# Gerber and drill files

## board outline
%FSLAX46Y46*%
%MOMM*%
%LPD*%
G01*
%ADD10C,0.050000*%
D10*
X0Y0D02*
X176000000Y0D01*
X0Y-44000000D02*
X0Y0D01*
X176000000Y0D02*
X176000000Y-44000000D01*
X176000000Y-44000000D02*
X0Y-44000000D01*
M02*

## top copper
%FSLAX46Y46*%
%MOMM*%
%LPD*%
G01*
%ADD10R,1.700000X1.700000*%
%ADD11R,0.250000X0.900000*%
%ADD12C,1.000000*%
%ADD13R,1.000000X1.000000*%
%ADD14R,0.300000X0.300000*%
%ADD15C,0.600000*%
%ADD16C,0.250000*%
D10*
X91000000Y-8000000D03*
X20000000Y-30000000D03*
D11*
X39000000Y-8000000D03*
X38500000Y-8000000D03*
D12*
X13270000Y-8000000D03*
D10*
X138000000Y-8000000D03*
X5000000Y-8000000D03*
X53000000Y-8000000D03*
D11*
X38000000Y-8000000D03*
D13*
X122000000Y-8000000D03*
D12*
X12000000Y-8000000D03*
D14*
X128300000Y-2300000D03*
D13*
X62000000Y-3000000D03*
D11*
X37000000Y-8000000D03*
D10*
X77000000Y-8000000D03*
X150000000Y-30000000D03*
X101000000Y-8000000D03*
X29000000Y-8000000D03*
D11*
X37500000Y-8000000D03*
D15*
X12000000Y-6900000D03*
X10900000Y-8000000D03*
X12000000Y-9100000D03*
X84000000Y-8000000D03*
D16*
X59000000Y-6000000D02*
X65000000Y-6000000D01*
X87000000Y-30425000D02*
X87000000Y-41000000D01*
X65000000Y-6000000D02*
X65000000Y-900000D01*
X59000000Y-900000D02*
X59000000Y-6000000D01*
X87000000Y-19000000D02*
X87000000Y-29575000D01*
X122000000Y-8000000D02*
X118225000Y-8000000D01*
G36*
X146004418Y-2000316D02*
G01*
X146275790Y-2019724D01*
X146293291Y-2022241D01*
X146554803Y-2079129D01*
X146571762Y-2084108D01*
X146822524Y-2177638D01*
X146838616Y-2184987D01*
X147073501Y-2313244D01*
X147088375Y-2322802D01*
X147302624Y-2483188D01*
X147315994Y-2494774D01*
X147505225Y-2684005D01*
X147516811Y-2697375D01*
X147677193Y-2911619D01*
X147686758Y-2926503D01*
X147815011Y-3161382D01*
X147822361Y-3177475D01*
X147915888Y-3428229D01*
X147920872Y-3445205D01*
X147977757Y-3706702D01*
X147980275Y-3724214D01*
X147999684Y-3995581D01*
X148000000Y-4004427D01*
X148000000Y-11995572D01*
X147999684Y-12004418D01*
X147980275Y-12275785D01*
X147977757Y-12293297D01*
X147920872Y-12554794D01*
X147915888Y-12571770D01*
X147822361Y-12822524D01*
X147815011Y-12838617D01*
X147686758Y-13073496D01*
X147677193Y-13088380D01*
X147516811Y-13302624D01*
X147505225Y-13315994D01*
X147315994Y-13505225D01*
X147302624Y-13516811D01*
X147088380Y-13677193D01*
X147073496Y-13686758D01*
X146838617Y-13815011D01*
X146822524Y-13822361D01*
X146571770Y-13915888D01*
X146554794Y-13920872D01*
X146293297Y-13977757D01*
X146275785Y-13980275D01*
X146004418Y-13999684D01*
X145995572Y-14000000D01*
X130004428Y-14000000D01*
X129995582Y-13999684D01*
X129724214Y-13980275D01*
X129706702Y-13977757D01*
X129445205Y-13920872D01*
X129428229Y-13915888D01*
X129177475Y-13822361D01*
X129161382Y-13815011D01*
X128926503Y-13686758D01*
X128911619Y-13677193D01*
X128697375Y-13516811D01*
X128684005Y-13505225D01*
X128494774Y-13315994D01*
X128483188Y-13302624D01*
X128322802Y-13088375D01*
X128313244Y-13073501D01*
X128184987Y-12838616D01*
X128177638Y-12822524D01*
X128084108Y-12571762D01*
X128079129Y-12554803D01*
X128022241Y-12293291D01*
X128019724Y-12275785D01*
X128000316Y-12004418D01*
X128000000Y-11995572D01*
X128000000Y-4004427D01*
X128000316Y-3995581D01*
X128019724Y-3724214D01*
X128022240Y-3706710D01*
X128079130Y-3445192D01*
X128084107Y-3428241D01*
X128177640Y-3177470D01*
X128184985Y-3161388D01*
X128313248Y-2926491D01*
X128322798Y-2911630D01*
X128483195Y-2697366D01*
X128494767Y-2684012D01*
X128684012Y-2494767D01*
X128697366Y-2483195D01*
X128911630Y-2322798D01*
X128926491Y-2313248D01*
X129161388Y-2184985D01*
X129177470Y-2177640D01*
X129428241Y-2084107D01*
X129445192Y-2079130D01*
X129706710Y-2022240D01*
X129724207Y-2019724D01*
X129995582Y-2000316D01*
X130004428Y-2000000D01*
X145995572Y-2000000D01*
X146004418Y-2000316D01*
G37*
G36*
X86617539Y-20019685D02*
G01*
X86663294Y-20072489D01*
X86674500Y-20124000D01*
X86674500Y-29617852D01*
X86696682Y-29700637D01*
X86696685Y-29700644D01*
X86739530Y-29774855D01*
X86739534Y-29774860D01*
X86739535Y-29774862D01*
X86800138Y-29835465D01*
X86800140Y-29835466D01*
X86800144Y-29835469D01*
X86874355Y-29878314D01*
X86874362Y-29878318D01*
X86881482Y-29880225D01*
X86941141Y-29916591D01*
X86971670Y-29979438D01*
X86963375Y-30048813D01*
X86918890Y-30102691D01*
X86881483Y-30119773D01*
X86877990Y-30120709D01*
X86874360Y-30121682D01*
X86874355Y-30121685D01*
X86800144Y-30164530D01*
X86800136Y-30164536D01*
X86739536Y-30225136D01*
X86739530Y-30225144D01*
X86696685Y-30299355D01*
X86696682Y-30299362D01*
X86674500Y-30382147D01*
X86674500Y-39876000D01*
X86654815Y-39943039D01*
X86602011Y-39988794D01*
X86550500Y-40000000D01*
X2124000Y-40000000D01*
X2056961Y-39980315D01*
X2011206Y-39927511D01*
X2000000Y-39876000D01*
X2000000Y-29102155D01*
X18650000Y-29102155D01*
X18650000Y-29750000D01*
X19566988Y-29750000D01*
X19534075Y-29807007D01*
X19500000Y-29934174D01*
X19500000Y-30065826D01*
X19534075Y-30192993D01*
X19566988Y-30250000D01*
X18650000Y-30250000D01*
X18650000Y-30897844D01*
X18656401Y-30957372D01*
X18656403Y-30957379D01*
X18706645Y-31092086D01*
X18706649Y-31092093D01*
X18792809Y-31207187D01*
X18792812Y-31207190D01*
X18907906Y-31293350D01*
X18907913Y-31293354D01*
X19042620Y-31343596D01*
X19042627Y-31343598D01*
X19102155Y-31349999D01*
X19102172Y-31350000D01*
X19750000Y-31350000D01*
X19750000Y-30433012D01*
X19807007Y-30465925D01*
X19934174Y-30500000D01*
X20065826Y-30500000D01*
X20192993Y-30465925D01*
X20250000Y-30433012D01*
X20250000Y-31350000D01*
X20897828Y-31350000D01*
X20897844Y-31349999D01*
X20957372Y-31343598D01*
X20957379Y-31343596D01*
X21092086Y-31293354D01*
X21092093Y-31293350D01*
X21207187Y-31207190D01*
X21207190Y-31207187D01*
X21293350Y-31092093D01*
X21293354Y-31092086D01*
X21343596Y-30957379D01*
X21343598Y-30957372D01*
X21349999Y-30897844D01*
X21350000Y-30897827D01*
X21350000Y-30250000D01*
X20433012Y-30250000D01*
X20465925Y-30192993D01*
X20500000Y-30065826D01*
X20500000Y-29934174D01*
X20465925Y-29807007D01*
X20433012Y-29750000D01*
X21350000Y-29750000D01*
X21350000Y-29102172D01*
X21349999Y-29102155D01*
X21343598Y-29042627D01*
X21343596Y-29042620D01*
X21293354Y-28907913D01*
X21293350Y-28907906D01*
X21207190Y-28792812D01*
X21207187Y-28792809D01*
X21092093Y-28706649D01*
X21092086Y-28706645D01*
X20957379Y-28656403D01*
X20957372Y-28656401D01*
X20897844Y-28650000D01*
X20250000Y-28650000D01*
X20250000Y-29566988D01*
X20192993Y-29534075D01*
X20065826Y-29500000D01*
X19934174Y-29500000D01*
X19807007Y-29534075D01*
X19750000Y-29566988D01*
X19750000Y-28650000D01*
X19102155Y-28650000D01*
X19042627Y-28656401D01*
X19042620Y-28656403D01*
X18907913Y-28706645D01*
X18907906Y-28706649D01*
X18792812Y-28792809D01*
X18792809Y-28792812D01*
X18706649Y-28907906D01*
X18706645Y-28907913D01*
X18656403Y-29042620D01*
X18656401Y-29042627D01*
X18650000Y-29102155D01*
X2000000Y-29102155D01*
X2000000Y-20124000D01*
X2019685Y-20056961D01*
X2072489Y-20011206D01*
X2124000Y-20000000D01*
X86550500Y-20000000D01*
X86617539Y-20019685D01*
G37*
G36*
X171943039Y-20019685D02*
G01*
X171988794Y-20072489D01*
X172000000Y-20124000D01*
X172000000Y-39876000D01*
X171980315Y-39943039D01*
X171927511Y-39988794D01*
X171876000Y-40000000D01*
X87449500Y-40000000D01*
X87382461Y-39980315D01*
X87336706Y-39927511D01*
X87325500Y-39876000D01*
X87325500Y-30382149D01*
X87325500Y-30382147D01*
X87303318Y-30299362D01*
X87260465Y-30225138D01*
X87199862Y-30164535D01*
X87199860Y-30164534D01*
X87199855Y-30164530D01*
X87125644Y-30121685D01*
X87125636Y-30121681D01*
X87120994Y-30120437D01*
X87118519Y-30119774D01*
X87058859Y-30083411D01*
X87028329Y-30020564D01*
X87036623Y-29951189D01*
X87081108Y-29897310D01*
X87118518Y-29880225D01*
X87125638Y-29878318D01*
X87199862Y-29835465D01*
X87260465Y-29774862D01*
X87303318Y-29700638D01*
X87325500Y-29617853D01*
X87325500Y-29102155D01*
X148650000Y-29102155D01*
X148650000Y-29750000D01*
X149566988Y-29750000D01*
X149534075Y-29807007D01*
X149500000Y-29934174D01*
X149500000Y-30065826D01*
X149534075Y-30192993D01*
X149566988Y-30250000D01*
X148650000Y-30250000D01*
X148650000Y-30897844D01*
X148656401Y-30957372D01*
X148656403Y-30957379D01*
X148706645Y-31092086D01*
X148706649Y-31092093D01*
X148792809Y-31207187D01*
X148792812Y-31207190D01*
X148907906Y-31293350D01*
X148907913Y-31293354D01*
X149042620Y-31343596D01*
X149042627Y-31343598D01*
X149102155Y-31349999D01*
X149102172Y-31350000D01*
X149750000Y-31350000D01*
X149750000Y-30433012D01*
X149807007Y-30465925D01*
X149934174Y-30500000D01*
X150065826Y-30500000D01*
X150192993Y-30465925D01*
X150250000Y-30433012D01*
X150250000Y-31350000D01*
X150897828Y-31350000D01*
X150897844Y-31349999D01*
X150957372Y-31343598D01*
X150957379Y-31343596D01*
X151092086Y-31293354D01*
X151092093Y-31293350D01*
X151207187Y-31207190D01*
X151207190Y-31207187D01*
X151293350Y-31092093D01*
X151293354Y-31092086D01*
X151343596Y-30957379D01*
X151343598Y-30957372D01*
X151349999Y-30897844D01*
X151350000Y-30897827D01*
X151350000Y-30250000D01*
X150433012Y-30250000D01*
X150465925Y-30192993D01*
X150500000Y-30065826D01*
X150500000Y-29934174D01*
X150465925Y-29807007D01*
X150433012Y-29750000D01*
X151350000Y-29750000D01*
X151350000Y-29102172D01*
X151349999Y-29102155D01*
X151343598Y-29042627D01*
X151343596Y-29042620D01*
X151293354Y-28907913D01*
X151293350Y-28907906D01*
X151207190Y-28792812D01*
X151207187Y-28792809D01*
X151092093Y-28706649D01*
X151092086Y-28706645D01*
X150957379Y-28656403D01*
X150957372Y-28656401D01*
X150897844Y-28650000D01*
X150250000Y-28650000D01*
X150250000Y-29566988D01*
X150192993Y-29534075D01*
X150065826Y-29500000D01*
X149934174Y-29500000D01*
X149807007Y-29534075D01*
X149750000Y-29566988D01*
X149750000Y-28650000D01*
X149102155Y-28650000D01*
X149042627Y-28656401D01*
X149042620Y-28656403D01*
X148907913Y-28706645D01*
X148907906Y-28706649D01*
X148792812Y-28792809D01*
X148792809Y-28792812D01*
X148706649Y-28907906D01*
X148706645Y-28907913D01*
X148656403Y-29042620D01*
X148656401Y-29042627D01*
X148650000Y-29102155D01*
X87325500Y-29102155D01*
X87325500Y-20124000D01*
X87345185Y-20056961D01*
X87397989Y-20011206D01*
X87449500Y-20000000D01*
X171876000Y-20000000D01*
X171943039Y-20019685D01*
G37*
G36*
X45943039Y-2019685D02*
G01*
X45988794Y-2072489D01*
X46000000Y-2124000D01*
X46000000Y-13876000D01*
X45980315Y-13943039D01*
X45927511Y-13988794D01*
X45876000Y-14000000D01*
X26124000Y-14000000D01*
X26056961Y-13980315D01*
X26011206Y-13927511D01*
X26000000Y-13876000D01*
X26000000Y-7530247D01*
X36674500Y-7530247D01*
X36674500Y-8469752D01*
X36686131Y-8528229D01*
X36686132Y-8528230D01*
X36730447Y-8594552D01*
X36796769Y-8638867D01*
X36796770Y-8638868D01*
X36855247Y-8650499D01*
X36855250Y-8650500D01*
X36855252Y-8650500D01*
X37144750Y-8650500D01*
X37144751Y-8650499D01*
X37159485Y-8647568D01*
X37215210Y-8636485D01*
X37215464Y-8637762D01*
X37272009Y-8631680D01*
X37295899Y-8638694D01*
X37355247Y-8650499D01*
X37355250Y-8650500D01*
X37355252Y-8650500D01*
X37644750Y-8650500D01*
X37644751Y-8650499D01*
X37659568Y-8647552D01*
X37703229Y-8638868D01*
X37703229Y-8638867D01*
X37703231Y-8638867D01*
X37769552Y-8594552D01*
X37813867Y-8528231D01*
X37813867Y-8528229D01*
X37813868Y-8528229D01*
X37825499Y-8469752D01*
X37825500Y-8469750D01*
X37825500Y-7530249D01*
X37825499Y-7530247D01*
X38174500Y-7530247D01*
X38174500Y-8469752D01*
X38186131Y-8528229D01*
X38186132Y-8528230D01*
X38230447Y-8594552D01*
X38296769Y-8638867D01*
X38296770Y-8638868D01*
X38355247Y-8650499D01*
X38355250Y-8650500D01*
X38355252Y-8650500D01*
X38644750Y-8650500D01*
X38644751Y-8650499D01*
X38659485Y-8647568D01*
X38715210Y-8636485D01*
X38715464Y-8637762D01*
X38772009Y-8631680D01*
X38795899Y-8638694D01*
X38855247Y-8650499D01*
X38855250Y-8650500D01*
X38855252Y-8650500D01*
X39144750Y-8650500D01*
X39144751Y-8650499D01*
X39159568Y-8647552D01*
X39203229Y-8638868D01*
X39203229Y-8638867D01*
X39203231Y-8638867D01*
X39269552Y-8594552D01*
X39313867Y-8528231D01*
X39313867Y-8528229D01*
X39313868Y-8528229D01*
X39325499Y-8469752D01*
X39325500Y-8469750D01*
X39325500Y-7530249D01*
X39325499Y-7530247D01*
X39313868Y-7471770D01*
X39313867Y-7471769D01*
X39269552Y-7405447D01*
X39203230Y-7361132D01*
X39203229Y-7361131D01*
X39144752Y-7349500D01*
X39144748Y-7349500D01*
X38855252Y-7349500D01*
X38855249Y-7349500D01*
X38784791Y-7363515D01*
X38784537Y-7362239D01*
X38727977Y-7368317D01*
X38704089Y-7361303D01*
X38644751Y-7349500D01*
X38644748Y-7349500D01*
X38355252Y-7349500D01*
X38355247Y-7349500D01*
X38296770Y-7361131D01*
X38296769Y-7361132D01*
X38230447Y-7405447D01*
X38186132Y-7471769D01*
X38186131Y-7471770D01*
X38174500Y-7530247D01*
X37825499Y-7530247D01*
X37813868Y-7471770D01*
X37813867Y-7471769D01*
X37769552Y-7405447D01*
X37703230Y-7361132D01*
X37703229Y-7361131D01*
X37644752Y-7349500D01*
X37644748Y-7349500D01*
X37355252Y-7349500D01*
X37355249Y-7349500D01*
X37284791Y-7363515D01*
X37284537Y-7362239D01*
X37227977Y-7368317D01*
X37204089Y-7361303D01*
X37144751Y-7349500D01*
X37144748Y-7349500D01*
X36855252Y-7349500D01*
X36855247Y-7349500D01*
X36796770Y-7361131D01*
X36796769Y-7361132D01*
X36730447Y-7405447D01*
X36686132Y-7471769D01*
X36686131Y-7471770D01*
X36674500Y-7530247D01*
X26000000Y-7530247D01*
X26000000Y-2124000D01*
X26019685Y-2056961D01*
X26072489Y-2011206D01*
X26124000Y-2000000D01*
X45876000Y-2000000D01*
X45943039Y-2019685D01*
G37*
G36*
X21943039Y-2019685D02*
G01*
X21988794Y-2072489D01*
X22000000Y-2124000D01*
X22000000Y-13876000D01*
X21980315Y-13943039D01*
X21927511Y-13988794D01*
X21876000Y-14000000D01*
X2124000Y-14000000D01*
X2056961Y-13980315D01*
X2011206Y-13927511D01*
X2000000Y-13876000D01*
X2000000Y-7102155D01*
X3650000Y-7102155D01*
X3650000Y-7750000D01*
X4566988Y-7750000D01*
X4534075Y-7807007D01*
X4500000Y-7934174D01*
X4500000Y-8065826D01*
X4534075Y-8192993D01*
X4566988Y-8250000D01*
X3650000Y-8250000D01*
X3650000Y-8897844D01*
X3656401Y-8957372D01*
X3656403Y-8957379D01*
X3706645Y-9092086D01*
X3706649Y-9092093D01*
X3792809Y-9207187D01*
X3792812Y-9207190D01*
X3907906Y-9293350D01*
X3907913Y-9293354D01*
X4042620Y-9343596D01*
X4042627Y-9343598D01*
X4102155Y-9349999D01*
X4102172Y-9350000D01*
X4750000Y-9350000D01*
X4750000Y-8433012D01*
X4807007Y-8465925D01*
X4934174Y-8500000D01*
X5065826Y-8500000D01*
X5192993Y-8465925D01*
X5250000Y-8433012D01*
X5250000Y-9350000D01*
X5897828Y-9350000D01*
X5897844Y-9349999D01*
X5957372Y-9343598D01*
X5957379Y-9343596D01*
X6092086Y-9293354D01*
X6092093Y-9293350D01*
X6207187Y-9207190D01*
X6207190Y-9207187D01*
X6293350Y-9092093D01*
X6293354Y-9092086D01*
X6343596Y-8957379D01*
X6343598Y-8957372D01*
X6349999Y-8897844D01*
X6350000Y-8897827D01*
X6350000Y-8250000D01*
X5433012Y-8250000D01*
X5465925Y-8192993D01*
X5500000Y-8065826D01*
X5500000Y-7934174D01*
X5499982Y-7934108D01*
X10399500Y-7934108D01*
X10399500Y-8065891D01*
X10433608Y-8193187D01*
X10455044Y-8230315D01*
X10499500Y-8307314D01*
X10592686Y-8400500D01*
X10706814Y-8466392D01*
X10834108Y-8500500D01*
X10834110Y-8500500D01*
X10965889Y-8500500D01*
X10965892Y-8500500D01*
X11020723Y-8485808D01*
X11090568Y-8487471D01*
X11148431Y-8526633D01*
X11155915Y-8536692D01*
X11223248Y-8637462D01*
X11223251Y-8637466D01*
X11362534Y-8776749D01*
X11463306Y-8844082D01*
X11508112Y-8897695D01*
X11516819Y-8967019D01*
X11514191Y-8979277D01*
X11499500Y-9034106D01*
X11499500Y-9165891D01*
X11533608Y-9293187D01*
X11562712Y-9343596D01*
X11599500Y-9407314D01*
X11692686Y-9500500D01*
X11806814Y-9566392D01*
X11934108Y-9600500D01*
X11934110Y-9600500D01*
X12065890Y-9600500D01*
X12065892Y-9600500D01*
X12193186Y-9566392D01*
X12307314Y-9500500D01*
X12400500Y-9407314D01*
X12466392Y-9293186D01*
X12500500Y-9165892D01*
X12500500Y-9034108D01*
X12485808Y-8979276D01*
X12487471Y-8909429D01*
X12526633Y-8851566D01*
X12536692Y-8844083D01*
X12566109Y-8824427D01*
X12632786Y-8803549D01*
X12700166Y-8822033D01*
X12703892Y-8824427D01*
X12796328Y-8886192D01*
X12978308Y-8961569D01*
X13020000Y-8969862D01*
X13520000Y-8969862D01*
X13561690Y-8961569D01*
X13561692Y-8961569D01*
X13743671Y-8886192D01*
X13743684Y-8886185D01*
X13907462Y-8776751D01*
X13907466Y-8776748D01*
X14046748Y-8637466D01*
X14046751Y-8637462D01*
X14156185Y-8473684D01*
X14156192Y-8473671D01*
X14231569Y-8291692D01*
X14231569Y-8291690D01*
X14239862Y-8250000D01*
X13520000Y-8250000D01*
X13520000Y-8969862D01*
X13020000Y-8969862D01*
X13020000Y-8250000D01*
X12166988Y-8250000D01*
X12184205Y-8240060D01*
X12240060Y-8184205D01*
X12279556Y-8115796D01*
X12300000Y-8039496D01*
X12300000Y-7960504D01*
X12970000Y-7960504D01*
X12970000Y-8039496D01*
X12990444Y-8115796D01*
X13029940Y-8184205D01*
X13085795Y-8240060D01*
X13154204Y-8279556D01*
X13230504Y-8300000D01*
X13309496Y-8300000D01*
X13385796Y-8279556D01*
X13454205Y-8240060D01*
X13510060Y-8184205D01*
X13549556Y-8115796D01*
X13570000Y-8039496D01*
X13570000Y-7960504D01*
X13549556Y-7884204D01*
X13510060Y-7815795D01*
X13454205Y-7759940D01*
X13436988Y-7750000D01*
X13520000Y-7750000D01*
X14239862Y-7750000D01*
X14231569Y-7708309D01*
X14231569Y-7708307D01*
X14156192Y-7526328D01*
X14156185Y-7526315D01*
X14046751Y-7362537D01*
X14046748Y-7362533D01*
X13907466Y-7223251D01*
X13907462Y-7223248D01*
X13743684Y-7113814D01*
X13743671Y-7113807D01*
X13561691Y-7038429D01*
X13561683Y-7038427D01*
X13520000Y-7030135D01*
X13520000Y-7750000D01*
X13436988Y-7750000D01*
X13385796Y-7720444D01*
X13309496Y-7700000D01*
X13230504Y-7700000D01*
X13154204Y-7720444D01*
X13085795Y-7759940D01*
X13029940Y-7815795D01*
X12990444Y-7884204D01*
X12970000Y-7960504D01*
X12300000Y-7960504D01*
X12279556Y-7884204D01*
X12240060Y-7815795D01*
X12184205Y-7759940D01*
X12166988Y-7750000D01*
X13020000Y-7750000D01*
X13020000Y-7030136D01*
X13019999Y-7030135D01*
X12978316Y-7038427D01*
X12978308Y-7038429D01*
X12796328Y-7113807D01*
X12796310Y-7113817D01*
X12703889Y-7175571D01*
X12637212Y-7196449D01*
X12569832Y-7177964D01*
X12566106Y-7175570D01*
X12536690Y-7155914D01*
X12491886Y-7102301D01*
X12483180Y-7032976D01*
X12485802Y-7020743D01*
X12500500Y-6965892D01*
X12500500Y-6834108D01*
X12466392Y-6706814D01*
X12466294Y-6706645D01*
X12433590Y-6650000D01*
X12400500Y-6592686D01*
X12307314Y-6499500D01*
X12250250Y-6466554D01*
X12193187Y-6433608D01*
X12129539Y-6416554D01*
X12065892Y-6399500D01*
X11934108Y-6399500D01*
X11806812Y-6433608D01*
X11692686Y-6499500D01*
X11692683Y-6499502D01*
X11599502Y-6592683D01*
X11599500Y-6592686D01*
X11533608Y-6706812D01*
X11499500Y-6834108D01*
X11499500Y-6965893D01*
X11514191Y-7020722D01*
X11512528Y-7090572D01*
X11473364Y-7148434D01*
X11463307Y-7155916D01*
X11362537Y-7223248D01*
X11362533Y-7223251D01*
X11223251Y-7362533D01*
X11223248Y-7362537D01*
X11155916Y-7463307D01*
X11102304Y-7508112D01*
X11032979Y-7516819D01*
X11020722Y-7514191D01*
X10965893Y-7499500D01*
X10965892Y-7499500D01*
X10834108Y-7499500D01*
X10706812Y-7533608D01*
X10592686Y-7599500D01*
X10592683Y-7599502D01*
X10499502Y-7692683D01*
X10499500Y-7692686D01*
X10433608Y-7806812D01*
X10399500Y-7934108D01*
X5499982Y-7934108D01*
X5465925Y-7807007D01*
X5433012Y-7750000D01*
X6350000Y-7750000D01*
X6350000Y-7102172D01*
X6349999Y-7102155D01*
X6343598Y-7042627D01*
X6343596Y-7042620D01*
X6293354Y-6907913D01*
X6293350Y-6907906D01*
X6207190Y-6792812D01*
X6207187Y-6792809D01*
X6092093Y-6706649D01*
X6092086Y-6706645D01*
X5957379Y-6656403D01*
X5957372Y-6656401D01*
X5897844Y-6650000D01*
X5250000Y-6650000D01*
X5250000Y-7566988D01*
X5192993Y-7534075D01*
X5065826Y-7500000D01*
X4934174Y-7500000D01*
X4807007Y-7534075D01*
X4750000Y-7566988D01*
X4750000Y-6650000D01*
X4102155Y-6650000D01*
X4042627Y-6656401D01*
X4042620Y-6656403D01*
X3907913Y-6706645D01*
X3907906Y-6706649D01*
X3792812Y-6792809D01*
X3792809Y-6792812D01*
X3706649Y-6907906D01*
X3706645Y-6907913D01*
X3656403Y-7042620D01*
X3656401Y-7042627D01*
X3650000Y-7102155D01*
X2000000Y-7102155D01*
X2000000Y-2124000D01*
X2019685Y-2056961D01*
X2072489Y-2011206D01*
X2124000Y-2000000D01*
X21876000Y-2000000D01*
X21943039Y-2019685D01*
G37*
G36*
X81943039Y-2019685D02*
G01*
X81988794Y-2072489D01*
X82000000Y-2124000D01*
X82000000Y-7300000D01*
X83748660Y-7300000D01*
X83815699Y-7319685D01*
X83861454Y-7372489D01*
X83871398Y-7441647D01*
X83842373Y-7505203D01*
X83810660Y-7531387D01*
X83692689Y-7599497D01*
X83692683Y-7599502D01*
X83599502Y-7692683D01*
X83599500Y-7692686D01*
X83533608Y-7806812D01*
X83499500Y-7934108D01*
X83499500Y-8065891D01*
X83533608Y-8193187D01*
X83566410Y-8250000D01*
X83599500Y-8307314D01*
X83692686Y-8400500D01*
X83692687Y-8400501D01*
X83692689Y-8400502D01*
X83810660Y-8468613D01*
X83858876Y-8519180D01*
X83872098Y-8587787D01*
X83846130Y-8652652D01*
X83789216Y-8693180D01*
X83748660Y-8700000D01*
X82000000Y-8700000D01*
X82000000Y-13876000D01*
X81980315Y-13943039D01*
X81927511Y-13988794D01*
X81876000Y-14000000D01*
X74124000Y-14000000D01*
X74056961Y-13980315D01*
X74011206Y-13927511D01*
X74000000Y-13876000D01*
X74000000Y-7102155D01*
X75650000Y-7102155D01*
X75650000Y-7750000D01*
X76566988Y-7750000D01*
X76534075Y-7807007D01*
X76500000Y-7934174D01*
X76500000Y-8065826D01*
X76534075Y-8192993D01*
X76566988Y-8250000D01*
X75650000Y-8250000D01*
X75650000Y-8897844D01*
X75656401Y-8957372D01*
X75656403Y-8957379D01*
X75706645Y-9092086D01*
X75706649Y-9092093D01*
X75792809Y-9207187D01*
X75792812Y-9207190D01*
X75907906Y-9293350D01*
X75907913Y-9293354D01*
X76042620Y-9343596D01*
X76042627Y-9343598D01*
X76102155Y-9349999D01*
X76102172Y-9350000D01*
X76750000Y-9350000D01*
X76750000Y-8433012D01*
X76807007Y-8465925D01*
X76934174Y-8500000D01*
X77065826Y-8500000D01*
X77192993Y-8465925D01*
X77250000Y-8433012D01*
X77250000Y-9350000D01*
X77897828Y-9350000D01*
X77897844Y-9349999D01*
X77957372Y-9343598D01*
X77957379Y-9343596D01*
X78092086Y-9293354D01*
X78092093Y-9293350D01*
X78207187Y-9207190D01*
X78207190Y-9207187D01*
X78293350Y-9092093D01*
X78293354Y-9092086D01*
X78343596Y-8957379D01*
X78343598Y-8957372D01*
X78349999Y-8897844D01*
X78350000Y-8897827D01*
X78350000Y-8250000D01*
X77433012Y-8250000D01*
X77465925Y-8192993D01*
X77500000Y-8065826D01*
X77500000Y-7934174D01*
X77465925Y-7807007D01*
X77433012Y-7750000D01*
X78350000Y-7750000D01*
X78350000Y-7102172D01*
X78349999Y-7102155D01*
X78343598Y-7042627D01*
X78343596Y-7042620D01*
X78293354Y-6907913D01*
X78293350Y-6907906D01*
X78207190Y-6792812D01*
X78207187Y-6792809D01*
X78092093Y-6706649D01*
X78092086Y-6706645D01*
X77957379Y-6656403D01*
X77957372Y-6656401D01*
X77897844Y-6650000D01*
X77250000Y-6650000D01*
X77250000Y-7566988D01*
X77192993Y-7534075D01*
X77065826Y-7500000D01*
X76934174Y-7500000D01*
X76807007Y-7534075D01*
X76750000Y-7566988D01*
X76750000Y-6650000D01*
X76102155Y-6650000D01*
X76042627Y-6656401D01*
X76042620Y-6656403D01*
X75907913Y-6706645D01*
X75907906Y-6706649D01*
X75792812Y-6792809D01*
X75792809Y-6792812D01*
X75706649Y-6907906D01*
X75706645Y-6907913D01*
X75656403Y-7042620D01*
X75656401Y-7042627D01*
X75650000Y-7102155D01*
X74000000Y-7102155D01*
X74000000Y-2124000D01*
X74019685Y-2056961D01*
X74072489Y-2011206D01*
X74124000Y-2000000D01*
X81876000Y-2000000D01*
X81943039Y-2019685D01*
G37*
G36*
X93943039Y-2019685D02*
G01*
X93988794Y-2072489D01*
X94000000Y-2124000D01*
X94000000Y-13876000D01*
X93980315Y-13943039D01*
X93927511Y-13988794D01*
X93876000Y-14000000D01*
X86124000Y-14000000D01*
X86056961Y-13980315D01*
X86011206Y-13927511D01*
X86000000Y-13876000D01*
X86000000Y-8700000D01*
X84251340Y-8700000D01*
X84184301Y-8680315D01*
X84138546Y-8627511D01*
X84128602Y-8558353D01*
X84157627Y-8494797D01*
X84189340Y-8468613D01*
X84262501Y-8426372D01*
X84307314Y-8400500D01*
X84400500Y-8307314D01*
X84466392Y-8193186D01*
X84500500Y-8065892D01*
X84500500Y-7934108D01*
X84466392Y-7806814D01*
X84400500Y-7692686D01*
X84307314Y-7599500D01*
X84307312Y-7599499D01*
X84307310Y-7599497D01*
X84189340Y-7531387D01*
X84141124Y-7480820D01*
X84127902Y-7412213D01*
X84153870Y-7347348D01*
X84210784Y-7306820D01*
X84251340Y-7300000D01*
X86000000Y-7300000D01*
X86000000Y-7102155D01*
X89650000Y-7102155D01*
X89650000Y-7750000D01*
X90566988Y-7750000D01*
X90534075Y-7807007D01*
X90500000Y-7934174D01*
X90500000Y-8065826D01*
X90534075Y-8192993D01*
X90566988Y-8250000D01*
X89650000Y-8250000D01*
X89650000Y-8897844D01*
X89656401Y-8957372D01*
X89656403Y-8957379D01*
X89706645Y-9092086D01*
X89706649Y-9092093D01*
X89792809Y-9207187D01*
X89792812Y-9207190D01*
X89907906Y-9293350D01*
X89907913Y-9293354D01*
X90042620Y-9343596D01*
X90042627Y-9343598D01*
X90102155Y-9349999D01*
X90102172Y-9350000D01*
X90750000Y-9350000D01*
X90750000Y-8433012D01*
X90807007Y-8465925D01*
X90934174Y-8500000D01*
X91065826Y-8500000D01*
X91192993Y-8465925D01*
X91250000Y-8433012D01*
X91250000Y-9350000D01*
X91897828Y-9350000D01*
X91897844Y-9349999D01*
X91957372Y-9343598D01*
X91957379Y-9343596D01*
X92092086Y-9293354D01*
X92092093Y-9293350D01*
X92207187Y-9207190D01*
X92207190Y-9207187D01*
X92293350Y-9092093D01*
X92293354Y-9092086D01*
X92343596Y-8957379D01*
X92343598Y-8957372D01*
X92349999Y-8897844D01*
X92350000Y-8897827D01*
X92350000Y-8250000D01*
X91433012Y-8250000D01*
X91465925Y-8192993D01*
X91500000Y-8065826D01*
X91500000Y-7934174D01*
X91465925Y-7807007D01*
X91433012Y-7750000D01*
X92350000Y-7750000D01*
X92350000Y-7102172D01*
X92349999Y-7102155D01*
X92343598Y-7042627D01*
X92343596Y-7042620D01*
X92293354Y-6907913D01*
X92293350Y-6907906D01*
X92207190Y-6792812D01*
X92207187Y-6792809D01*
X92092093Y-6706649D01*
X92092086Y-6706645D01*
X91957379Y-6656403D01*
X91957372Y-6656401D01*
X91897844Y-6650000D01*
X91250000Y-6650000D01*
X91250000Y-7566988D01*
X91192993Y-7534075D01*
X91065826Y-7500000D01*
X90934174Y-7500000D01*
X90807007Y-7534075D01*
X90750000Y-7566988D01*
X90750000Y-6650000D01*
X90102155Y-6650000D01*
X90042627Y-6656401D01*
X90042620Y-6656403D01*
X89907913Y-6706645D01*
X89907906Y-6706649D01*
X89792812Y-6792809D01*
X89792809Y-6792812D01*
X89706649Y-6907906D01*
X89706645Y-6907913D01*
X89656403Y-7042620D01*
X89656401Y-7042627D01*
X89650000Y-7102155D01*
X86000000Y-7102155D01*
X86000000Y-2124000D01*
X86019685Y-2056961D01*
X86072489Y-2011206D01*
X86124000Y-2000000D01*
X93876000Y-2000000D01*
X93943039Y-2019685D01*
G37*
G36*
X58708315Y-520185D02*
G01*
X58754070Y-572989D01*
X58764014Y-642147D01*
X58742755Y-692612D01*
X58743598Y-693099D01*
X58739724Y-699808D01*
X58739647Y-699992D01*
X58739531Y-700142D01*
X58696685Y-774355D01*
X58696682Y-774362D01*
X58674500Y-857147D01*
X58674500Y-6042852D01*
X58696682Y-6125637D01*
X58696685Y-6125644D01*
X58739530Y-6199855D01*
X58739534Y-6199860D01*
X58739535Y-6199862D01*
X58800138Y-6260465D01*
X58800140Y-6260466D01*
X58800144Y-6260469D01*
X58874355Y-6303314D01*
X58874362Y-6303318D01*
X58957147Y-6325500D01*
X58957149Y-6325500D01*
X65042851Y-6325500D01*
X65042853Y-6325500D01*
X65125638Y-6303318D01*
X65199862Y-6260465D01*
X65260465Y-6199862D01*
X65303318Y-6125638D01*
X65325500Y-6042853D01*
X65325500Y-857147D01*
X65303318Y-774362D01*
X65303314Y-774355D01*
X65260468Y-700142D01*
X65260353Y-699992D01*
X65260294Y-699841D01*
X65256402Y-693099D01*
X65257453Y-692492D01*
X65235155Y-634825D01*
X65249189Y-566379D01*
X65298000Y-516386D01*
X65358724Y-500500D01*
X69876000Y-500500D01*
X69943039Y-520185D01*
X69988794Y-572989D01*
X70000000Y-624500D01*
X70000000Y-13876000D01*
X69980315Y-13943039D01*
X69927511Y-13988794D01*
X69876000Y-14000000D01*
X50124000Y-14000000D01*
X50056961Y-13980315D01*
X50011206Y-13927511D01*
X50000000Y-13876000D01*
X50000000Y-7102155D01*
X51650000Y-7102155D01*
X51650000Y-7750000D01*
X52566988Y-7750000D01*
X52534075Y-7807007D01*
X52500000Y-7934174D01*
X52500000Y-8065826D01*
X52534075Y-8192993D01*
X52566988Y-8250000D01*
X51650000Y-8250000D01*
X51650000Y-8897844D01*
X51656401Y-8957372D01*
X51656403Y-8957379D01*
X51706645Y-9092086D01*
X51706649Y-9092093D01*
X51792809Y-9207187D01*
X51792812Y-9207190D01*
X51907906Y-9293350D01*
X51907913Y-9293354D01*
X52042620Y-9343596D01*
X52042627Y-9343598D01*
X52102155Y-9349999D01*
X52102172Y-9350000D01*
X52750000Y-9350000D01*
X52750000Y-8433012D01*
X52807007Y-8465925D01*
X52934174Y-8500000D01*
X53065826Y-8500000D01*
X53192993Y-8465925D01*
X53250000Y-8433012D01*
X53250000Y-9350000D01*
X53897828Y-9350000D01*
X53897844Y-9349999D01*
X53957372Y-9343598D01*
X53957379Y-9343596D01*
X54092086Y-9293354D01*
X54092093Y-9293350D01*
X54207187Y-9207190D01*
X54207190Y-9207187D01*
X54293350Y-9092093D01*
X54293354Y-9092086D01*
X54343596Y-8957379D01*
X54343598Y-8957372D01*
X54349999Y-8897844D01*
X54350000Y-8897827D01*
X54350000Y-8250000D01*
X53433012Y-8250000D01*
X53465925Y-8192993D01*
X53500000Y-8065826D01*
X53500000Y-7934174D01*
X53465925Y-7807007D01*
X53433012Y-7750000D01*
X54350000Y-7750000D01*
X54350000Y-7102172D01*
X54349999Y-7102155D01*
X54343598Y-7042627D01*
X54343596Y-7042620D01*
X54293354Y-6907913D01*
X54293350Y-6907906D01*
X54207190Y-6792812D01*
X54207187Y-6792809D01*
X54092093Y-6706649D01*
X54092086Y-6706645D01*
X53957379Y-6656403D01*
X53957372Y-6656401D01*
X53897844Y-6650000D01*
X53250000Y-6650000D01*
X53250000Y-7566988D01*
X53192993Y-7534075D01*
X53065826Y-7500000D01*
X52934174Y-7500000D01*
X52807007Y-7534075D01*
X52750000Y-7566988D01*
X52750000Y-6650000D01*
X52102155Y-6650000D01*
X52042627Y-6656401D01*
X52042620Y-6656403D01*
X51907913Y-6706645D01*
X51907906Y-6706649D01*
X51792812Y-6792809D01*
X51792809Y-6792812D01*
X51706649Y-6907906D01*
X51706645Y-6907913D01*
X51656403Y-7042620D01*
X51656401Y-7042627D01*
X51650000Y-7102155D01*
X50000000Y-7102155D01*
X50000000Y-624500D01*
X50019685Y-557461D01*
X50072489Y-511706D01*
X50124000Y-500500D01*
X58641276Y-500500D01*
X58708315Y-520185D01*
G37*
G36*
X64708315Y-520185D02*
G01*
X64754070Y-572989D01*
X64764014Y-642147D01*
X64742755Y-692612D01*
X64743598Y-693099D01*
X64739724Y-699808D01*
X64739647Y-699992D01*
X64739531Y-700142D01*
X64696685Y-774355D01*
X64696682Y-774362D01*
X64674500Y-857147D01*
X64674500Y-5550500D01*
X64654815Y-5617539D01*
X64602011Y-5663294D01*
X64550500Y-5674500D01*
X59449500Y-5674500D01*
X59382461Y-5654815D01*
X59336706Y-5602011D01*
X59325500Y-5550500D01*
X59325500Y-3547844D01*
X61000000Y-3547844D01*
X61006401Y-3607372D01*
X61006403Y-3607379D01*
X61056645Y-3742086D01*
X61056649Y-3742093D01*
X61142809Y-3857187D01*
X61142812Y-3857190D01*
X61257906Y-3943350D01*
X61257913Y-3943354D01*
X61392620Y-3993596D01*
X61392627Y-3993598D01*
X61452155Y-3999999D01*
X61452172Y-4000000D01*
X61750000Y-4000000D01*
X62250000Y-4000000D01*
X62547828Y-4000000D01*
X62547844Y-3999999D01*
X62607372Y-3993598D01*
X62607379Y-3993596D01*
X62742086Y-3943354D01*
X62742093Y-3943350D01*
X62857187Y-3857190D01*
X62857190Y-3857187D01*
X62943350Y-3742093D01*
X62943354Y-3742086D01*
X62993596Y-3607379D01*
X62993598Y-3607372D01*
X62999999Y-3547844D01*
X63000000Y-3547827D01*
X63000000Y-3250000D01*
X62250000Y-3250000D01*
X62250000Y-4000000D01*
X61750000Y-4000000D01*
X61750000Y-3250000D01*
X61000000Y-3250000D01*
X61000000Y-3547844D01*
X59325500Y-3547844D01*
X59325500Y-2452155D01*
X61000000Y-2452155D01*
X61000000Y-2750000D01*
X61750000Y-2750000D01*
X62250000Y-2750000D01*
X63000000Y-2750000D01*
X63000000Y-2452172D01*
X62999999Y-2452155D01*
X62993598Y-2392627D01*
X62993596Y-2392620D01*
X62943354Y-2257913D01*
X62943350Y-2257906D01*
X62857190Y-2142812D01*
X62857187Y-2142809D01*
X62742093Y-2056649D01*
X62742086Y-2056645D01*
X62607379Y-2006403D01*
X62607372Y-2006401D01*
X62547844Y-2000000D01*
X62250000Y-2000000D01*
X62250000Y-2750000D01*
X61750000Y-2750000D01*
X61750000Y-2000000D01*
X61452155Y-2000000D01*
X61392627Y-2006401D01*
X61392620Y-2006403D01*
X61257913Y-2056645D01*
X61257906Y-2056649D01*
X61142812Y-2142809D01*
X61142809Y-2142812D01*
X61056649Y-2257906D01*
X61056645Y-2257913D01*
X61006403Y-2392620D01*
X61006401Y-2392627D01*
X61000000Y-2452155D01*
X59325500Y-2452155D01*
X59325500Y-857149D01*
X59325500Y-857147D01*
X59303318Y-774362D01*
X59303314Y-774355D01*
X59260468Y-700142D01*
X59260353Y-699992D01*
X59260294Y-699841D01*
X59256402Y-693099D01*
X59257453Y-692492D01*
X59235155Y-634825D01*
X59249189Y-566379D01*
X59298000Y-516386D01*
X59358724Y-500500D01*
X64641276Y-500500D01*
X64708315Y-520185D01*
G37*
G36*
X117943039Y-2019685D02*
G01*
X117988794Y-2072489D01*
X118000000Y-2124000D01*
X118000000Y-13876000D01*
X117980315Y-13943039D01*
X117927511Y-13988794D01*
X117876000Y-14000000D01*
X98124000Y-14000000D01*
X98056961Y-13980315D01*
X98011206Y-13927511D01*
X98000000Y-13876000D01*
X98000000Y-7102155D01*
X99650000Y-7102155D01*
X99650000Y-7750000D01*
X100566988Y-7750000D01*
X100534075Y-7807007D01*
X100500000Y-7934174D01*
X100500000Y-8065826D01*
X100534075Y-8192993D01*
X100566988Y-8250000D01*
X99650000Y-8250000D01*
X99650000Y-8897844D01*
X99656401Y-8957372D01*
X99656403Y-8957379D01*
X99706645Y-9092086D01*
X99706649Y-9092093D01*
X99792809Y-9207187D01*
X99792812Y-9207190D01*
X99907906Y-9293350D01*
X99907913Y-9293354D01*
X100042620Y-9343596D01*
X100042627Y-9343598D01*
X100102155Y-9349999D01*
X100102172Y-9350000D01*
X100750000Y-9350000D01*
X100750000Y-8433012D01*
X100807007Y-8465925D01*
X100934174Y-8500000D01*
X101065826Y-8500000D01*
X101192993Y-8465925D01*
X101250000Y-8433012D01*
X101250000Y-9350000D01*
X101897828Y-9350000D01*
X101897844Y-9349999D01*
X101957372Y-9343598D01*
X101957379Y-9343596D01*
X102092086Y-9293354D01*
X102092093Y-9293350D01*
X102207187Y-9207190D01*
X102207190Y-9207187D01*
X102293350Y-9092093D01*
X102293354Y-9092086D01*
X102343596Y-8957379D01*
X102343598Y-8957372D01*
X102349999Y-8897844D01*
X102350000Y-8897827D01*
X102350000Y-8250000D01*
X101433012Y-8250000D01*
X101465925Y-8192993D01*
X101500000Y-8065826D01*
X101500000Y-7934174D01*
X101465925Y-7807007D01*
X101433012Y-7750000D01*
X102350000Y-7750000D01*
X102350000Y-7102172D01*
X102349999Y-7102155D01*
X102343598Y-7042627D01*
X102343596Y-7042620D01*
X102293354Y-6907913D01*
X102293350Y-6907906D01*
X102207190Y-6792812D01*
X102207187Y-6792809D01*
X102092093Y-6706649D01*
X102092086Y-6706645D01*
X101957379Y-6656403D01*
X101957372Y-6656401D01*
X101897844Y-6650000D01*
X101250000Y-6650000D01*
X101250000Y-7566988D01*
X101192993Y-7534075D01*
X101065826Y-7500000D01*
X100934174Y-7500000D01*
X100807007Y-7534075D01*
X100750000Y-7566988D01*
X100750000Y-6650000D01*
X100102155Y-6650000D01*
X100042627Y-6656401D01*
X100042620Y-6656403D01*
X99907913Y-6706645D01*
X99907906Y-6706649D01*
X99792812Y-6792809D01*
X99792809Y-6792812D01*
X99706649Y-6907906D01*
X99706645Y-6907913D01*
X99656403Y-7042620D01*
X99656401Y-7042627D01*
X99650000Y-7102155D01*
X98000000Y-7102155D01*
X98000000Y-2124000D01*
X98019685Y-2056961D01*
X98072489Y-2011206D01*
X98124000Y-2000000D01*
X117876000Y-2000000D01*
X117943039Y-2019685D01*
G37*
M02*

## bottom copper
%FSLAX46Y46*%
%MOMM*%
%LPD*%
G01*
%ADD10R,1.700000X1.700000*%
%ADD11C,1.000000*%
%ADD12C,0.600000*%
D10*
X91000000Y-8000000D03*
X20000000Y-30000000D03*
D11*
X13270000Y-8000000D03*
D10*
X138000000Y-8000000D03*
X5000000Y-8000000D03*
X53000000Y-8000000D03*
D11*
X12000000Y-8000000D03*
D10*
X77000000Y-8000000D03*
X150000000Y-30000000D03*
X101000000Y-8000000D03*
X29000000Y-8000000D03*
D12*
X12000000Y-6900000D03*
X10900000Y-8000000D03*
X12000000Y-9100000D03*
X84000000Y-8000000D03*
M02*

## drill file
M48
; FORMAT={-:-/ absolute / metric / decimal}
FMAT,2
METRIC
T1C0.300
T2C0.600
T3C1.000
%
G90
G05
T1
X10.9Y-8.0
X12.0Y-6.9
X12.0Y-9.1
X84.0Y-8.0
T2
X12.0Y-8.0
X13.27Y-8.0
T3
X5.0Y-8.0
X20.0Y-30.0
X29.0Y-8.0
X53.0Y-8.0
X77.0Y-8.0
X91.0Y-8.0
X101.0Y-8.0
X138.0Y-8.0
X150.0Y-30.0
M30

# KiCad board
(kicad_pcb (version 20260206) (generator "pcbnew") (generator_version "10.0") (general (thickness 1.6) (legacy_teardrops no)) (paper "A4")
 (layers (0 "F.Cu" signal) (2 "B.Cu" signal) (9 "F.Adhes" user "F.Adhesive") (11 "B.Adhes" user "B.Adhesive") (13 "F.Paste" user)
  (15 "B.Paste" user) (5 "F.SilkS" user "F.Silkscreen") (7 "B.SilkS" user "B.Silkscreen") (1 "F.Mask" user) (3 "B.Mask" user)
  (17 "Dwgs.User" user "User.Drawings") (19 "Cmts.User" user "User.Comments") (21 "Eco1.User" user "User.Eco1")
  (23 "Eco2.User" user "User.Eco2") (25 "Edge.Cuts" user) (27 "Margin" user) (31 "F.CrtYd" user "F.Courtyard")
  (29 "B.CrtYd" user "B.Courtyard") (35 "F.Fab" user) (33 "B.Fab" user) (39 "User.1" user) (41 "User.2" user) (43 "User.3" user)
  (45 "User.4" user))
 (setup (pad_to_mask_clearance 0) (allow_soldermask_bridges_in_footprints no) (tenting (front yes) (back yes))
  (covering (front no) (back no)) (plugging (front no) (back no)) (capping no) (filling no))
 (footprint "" (layer "F.Cu") (at 91 8)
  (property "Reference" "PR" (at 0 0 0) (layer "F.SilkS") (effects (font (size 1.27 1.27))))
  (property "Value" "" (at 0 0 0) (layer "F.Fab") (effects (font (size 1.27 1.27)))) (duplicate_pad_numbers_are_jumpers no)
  (pad "1" thru_hole rect (at 0 0) (size 1.7 1.7) (drill 1) (layers "*.Cu" "*.Mask") (remove_unused_layers no) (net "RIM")))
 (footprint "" (layer "F.Cu") (at 20 30)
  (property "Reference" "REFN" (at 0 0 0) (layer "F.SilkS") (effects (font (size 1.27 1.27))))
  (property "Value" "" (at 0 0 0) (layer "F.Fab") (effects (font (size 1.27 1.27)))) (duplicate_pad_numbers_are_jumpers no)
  (pad "1" thru_hole rect (at 0 0) (size 1.7 1.7) (drill 1) (layers "*.Cu" "*.Mask") (remove_unused_layers no) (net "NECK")))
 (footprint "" (layer "F.Cu") (at 39 8)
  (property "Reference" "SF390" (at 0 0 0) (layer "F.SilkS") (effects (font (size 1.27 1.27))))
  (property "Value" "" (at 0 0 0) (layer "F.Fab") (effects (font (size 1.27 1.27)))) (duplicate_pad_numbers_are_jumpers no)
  (pad "1" smd rect (at 0 0) (size 0.25 0.9) (layers "F.Cu" "F.Mask" "F.Paste") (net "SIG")))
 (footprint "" (layer "F.Cu") (at 38.5 8)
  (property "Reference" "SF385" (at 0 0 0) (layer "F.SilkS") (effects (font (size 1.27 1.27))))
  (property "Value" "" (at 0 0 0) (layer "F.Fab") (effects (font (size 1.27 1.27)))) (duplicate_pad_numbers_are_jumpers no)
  (pad "1" smd rect (at 0 0) (size 0.25 0.9) (layers "F.Cu" "F.Mask" "F.Paste") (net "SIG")))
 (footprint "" (layer "F.Cu") (at 13.27 8)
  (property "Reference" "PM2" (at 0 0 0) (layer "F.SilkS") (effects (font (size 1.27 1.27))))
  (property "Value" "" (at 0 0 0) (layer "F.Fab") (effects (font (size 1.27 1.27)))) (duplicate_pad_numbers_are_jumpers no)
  (pad "1" thru_hole circle (at 0 0) (size 1 1) (drill 0.6) (layers "*.Cu" "*.Mask") (remove_unused_layers no) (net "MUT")
   (thermal_bridge_angle 90)))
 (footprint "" (layer "F.Cu") (at 138 8)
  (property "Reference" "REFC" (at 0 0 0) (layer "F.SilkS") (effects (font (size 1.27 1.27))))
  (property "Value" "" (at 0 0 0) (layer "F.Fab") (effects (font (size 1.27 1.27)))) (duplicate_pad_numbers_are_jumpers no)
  (pad "1" thru_hole rect (at 0 0) (size 1.7 1.7) (drill 1) (layers "*.Cu" "*.Mask") (remove_unused_layers no) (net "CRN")))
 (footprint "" (layer "F.Cu") (at 5 8)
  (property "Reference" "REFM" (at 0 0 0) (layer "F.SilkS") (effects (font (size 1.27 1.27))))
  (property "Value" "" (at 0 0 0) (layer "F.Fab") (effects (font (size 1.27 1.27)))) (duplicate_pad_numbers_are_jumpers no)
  (pad "1" thru_hole rect (at 0 0) (size 1.7 1.7) (drill 1) (layers "*.Cu" "*.Mask") (remove_unused_layers no) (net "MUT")))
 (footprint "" (layer "F.Cu") (at 53 8)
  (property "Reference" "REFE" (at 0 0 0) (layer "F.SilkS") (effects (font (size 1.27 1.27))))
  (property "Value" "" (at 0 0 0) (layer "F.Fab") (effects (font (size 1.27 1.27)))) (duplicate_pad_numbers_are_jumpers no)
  (pad "1" thru_hole rect (at 0 0) (size 1.7 1.7) (drill 1) (layers "*.Cu" "*.Mask") (remove_unused_layers no) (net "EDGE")))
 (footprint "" (layer "F.Cu") (at 38 8)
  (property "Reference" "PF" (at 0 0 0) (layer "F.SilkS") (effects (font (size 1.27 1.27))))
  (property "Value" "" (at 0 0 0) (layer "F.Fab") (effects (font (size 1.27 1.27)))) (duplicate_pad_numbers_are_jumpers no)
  (pad "1" smd rect (at 0 0) (size 0.25 0.9) (layers "F.Cu" "F.Mask" "F.Paste") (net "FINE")))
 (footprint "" (layer "F.Cu") (at 122 8)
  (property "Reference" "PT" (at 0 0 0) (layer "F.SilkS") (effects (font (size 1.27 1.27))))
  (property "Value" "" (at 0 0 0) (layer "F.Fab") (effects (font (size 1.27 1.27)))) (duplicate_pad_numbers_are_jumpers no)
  (pad "1" smd rect (at 0 0) (size 1 1) (layers "F.Cu" "F.Mask" "F.Paste") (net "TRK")))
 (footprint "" (layer "F.Cu") (at 12 8)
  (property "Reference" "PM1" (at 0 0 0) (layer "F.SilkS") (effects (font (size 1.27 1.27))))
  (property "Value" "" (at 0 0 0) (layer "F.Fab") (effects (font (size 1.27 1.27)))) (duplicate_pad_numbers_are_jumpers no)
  (pad "1" thru_hole circle (at 0 0) (size 1 1) (drill 0.6) (layers "*.Cu" "*.Mask") (remove_unused_layers no) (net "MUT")
   (thermal_bridge_angle 90)))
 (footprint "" (layer "F.Cu") (at 128.3 2.3)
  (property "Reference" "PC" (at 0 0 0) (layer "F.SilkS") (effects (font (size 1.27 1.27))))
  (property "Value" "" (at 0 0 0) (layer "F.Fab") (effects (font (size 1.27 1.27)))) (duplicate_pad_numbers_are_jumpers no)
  (pad "1" smd rect (at 0 0) (size 0.3 0.3) (layers "F.Cu" "F.Mask" "F.Paste") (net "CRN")))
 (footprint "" (layer "F.Cu") (at 62 3)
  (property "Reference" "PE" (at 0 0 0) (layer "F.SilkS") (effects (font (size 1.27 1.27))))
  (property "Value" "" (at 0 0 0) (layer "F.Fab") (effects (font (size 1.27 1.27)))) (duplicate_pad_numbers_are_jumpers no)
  (pad "1" smd rect (at 0 0) (size 1 1) (layers "F.Cu" "F.Mask" "F.Paste") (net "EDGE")))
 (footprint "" (layer "F.Cu") (at 37 8)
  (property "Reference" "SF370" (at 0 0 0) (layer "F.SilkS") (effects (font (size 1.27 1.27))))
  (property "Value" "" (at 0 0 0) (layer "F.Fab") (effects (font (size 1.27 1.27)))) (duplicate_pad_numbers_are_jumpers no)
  (pad "1" smd rect (at 0 0) (size 0.25 0.9) (layers "F.Cu" "F.Mask" "F.Paste") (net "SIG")))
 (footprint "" (layer "F.Cu") (at 77 8)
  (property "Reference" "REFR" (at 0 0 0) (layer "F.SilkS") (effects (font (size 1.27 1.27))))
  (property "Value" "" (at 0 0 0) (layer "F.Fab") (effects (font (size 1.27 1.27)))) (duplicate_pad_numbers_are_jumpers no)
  (pad "1" thru_hole rect (at 0 0) (size 1.7 1.7) (drill 1) (layers "*.Cu" "*.Mask") (remove_unused_layers no) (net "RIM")))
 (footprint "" (layer "F.Cu") (at 150 30)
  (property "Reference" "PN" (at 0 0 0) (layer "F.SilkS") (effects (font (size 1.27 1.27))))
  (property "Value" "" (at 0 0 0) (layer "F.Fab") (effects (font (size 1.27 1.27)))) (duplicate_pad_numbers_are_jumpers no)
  (pad "1" thru_hole rect (at 0 0) (size 1.7 1.7) (drill 1) (layers "*.Cu" "*.Mask") (remove_unused_layers no) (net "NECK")))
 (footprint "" (layer "F.Cu") (at 101 8)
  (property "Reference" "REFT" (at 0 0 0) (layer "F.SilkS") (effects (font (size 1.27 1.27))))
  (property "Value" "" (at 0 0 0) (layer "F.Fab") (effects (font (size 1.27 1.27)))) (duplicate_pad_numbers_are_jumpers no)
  (pad "1" thru_hole rect (at 0 0) (size 1.7 1.7) (drill 1) (layers "*.Cu" "*.Mask") (remove_unused_layers no) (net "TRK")))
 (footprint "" (layer "F.Cu") (at 29 8)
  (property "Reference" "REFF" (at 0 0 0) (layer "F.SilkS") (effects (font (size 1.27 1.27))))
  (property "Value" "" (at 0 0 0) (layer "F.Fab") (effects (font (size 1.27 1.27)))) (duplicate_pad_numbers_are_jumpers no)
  (pad "1" thru_hole rect (at 0 0) (size 1.7 1.7) (drill 1) (layers "*.Cu" "*.Mask") (remove_unused_layers no) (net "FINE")))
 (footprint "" (layer "F.Cu") (at 37.5 8)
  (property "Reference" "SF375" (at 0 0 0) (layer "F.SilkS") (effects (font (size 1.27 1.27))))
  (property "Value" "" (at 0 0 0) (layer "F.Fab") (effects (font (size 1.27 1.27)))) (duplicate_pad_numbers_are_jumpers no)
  (pad "1" smd rect (at 0 0) (size 0.25 0.9) (layers "F.Cu" "F.Mask" "F.Paste") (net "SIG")))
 (gr_line (start 0 0) (end 176 0) (stroke (width 0.05) (type default)) (layer "Edge.Cuts"))
 (gr_line (start 0 44) (end 0 0) (stroke (width 0.05) (type default)) (layer "Edge.Cuts"))
 (gr_line (start 176 0) (end 176 44) (stroke (width 0.05) (type default)) (layer "Edge.Cuts"))
 (gr_line (start 176 44) (end 0 44) (stroke (width 0.05) (type default)) (layer "Edge.Cuts"))
 (segment (start 59 6) (end 65 6) (width 0.25) (layer "F.Cu") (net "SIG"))
 (segment (start 87 30.425) (end 87 41) (width 0.25) (layer "F.Cu") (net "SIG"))
 (segment (start 65 6) (end 65 0.9) (width 0.25) (layer "F.Cu") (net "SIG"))
 (segment (start 59 0.9) (end 59 6) (width 0.25) (layer "F.Cu") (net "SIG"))
 (segment (start 87 19) (end 87 29.575) (width 0.25) (layer "F.Cu") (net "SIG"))
 (via (at 12 6.9) (size 0.6) (drill 0.3) (layers "F.Cu" "B.Cu") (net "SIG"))
 (via (at 10.9 8) (size 0.6) (drill 0.3) (layers "F.Cu" "B.Cu") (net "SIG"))
 (via (at 12 9.1) (size 0.6) (drill 0.3) (layers "F.Cu" "B.Cu") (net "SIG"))
 (via (at 84 8) (size 0.6) (drill 0.3) (layers "F.Cu" "B.Cu") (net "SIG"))
 (segment (start 122 8) (end 118.225 8) (width 0.25) (layer "F.Cu") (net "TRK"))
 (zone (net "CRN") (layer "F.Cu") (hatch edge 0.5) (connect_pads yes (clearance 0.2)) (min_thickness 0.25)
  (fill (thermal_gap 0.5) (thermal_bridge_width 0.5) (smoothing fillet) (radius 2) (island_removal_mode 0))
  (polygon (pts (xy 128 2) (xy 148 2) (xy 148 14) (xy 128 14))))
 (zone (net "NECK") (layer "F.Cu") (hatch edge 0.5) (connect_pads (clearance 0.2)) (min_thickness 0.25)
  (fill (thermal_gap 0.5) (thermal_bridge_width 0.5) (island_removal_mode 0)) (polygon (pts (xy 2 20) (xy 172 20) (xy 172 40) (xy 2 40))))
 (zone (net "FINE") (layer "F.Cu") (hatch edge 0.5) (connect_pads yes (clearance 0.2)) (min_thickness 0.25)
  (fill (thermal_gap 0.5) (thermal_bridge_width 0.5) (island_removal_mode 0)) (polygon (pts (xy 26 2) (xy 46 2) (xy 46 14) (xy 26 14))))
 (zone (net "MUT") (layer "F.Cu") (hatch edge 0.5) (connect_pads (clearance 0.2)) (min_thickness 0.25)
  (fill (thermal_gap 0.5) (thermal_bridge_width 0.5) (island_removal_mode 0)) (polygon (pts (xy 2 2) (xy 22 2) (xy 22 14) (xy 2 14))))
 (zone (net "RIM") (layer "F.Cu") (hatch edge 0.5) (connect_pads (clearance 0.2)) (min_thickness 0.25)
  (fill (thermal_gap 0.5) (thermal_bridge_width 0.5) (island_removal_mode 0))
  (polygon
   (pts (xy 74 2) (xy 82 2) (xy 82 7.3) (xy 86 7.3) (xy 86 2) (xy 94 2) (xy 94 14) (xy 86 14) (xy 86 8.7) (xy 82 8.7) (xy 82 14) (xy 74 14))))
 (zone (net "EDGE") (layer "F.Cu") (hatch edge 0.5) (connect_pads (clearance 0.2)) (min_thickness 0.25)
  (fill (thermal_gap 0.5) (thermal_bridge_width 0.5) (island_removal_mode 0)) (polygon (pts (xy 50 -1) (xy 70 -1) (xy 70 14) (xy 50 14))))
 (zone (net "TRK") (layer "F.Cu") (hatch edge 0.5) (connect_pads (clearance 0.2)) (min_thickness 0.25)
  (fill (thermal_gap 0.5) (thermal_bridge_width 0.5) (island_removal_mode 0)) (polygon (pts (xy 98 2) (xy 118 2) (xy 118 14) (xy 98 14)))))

